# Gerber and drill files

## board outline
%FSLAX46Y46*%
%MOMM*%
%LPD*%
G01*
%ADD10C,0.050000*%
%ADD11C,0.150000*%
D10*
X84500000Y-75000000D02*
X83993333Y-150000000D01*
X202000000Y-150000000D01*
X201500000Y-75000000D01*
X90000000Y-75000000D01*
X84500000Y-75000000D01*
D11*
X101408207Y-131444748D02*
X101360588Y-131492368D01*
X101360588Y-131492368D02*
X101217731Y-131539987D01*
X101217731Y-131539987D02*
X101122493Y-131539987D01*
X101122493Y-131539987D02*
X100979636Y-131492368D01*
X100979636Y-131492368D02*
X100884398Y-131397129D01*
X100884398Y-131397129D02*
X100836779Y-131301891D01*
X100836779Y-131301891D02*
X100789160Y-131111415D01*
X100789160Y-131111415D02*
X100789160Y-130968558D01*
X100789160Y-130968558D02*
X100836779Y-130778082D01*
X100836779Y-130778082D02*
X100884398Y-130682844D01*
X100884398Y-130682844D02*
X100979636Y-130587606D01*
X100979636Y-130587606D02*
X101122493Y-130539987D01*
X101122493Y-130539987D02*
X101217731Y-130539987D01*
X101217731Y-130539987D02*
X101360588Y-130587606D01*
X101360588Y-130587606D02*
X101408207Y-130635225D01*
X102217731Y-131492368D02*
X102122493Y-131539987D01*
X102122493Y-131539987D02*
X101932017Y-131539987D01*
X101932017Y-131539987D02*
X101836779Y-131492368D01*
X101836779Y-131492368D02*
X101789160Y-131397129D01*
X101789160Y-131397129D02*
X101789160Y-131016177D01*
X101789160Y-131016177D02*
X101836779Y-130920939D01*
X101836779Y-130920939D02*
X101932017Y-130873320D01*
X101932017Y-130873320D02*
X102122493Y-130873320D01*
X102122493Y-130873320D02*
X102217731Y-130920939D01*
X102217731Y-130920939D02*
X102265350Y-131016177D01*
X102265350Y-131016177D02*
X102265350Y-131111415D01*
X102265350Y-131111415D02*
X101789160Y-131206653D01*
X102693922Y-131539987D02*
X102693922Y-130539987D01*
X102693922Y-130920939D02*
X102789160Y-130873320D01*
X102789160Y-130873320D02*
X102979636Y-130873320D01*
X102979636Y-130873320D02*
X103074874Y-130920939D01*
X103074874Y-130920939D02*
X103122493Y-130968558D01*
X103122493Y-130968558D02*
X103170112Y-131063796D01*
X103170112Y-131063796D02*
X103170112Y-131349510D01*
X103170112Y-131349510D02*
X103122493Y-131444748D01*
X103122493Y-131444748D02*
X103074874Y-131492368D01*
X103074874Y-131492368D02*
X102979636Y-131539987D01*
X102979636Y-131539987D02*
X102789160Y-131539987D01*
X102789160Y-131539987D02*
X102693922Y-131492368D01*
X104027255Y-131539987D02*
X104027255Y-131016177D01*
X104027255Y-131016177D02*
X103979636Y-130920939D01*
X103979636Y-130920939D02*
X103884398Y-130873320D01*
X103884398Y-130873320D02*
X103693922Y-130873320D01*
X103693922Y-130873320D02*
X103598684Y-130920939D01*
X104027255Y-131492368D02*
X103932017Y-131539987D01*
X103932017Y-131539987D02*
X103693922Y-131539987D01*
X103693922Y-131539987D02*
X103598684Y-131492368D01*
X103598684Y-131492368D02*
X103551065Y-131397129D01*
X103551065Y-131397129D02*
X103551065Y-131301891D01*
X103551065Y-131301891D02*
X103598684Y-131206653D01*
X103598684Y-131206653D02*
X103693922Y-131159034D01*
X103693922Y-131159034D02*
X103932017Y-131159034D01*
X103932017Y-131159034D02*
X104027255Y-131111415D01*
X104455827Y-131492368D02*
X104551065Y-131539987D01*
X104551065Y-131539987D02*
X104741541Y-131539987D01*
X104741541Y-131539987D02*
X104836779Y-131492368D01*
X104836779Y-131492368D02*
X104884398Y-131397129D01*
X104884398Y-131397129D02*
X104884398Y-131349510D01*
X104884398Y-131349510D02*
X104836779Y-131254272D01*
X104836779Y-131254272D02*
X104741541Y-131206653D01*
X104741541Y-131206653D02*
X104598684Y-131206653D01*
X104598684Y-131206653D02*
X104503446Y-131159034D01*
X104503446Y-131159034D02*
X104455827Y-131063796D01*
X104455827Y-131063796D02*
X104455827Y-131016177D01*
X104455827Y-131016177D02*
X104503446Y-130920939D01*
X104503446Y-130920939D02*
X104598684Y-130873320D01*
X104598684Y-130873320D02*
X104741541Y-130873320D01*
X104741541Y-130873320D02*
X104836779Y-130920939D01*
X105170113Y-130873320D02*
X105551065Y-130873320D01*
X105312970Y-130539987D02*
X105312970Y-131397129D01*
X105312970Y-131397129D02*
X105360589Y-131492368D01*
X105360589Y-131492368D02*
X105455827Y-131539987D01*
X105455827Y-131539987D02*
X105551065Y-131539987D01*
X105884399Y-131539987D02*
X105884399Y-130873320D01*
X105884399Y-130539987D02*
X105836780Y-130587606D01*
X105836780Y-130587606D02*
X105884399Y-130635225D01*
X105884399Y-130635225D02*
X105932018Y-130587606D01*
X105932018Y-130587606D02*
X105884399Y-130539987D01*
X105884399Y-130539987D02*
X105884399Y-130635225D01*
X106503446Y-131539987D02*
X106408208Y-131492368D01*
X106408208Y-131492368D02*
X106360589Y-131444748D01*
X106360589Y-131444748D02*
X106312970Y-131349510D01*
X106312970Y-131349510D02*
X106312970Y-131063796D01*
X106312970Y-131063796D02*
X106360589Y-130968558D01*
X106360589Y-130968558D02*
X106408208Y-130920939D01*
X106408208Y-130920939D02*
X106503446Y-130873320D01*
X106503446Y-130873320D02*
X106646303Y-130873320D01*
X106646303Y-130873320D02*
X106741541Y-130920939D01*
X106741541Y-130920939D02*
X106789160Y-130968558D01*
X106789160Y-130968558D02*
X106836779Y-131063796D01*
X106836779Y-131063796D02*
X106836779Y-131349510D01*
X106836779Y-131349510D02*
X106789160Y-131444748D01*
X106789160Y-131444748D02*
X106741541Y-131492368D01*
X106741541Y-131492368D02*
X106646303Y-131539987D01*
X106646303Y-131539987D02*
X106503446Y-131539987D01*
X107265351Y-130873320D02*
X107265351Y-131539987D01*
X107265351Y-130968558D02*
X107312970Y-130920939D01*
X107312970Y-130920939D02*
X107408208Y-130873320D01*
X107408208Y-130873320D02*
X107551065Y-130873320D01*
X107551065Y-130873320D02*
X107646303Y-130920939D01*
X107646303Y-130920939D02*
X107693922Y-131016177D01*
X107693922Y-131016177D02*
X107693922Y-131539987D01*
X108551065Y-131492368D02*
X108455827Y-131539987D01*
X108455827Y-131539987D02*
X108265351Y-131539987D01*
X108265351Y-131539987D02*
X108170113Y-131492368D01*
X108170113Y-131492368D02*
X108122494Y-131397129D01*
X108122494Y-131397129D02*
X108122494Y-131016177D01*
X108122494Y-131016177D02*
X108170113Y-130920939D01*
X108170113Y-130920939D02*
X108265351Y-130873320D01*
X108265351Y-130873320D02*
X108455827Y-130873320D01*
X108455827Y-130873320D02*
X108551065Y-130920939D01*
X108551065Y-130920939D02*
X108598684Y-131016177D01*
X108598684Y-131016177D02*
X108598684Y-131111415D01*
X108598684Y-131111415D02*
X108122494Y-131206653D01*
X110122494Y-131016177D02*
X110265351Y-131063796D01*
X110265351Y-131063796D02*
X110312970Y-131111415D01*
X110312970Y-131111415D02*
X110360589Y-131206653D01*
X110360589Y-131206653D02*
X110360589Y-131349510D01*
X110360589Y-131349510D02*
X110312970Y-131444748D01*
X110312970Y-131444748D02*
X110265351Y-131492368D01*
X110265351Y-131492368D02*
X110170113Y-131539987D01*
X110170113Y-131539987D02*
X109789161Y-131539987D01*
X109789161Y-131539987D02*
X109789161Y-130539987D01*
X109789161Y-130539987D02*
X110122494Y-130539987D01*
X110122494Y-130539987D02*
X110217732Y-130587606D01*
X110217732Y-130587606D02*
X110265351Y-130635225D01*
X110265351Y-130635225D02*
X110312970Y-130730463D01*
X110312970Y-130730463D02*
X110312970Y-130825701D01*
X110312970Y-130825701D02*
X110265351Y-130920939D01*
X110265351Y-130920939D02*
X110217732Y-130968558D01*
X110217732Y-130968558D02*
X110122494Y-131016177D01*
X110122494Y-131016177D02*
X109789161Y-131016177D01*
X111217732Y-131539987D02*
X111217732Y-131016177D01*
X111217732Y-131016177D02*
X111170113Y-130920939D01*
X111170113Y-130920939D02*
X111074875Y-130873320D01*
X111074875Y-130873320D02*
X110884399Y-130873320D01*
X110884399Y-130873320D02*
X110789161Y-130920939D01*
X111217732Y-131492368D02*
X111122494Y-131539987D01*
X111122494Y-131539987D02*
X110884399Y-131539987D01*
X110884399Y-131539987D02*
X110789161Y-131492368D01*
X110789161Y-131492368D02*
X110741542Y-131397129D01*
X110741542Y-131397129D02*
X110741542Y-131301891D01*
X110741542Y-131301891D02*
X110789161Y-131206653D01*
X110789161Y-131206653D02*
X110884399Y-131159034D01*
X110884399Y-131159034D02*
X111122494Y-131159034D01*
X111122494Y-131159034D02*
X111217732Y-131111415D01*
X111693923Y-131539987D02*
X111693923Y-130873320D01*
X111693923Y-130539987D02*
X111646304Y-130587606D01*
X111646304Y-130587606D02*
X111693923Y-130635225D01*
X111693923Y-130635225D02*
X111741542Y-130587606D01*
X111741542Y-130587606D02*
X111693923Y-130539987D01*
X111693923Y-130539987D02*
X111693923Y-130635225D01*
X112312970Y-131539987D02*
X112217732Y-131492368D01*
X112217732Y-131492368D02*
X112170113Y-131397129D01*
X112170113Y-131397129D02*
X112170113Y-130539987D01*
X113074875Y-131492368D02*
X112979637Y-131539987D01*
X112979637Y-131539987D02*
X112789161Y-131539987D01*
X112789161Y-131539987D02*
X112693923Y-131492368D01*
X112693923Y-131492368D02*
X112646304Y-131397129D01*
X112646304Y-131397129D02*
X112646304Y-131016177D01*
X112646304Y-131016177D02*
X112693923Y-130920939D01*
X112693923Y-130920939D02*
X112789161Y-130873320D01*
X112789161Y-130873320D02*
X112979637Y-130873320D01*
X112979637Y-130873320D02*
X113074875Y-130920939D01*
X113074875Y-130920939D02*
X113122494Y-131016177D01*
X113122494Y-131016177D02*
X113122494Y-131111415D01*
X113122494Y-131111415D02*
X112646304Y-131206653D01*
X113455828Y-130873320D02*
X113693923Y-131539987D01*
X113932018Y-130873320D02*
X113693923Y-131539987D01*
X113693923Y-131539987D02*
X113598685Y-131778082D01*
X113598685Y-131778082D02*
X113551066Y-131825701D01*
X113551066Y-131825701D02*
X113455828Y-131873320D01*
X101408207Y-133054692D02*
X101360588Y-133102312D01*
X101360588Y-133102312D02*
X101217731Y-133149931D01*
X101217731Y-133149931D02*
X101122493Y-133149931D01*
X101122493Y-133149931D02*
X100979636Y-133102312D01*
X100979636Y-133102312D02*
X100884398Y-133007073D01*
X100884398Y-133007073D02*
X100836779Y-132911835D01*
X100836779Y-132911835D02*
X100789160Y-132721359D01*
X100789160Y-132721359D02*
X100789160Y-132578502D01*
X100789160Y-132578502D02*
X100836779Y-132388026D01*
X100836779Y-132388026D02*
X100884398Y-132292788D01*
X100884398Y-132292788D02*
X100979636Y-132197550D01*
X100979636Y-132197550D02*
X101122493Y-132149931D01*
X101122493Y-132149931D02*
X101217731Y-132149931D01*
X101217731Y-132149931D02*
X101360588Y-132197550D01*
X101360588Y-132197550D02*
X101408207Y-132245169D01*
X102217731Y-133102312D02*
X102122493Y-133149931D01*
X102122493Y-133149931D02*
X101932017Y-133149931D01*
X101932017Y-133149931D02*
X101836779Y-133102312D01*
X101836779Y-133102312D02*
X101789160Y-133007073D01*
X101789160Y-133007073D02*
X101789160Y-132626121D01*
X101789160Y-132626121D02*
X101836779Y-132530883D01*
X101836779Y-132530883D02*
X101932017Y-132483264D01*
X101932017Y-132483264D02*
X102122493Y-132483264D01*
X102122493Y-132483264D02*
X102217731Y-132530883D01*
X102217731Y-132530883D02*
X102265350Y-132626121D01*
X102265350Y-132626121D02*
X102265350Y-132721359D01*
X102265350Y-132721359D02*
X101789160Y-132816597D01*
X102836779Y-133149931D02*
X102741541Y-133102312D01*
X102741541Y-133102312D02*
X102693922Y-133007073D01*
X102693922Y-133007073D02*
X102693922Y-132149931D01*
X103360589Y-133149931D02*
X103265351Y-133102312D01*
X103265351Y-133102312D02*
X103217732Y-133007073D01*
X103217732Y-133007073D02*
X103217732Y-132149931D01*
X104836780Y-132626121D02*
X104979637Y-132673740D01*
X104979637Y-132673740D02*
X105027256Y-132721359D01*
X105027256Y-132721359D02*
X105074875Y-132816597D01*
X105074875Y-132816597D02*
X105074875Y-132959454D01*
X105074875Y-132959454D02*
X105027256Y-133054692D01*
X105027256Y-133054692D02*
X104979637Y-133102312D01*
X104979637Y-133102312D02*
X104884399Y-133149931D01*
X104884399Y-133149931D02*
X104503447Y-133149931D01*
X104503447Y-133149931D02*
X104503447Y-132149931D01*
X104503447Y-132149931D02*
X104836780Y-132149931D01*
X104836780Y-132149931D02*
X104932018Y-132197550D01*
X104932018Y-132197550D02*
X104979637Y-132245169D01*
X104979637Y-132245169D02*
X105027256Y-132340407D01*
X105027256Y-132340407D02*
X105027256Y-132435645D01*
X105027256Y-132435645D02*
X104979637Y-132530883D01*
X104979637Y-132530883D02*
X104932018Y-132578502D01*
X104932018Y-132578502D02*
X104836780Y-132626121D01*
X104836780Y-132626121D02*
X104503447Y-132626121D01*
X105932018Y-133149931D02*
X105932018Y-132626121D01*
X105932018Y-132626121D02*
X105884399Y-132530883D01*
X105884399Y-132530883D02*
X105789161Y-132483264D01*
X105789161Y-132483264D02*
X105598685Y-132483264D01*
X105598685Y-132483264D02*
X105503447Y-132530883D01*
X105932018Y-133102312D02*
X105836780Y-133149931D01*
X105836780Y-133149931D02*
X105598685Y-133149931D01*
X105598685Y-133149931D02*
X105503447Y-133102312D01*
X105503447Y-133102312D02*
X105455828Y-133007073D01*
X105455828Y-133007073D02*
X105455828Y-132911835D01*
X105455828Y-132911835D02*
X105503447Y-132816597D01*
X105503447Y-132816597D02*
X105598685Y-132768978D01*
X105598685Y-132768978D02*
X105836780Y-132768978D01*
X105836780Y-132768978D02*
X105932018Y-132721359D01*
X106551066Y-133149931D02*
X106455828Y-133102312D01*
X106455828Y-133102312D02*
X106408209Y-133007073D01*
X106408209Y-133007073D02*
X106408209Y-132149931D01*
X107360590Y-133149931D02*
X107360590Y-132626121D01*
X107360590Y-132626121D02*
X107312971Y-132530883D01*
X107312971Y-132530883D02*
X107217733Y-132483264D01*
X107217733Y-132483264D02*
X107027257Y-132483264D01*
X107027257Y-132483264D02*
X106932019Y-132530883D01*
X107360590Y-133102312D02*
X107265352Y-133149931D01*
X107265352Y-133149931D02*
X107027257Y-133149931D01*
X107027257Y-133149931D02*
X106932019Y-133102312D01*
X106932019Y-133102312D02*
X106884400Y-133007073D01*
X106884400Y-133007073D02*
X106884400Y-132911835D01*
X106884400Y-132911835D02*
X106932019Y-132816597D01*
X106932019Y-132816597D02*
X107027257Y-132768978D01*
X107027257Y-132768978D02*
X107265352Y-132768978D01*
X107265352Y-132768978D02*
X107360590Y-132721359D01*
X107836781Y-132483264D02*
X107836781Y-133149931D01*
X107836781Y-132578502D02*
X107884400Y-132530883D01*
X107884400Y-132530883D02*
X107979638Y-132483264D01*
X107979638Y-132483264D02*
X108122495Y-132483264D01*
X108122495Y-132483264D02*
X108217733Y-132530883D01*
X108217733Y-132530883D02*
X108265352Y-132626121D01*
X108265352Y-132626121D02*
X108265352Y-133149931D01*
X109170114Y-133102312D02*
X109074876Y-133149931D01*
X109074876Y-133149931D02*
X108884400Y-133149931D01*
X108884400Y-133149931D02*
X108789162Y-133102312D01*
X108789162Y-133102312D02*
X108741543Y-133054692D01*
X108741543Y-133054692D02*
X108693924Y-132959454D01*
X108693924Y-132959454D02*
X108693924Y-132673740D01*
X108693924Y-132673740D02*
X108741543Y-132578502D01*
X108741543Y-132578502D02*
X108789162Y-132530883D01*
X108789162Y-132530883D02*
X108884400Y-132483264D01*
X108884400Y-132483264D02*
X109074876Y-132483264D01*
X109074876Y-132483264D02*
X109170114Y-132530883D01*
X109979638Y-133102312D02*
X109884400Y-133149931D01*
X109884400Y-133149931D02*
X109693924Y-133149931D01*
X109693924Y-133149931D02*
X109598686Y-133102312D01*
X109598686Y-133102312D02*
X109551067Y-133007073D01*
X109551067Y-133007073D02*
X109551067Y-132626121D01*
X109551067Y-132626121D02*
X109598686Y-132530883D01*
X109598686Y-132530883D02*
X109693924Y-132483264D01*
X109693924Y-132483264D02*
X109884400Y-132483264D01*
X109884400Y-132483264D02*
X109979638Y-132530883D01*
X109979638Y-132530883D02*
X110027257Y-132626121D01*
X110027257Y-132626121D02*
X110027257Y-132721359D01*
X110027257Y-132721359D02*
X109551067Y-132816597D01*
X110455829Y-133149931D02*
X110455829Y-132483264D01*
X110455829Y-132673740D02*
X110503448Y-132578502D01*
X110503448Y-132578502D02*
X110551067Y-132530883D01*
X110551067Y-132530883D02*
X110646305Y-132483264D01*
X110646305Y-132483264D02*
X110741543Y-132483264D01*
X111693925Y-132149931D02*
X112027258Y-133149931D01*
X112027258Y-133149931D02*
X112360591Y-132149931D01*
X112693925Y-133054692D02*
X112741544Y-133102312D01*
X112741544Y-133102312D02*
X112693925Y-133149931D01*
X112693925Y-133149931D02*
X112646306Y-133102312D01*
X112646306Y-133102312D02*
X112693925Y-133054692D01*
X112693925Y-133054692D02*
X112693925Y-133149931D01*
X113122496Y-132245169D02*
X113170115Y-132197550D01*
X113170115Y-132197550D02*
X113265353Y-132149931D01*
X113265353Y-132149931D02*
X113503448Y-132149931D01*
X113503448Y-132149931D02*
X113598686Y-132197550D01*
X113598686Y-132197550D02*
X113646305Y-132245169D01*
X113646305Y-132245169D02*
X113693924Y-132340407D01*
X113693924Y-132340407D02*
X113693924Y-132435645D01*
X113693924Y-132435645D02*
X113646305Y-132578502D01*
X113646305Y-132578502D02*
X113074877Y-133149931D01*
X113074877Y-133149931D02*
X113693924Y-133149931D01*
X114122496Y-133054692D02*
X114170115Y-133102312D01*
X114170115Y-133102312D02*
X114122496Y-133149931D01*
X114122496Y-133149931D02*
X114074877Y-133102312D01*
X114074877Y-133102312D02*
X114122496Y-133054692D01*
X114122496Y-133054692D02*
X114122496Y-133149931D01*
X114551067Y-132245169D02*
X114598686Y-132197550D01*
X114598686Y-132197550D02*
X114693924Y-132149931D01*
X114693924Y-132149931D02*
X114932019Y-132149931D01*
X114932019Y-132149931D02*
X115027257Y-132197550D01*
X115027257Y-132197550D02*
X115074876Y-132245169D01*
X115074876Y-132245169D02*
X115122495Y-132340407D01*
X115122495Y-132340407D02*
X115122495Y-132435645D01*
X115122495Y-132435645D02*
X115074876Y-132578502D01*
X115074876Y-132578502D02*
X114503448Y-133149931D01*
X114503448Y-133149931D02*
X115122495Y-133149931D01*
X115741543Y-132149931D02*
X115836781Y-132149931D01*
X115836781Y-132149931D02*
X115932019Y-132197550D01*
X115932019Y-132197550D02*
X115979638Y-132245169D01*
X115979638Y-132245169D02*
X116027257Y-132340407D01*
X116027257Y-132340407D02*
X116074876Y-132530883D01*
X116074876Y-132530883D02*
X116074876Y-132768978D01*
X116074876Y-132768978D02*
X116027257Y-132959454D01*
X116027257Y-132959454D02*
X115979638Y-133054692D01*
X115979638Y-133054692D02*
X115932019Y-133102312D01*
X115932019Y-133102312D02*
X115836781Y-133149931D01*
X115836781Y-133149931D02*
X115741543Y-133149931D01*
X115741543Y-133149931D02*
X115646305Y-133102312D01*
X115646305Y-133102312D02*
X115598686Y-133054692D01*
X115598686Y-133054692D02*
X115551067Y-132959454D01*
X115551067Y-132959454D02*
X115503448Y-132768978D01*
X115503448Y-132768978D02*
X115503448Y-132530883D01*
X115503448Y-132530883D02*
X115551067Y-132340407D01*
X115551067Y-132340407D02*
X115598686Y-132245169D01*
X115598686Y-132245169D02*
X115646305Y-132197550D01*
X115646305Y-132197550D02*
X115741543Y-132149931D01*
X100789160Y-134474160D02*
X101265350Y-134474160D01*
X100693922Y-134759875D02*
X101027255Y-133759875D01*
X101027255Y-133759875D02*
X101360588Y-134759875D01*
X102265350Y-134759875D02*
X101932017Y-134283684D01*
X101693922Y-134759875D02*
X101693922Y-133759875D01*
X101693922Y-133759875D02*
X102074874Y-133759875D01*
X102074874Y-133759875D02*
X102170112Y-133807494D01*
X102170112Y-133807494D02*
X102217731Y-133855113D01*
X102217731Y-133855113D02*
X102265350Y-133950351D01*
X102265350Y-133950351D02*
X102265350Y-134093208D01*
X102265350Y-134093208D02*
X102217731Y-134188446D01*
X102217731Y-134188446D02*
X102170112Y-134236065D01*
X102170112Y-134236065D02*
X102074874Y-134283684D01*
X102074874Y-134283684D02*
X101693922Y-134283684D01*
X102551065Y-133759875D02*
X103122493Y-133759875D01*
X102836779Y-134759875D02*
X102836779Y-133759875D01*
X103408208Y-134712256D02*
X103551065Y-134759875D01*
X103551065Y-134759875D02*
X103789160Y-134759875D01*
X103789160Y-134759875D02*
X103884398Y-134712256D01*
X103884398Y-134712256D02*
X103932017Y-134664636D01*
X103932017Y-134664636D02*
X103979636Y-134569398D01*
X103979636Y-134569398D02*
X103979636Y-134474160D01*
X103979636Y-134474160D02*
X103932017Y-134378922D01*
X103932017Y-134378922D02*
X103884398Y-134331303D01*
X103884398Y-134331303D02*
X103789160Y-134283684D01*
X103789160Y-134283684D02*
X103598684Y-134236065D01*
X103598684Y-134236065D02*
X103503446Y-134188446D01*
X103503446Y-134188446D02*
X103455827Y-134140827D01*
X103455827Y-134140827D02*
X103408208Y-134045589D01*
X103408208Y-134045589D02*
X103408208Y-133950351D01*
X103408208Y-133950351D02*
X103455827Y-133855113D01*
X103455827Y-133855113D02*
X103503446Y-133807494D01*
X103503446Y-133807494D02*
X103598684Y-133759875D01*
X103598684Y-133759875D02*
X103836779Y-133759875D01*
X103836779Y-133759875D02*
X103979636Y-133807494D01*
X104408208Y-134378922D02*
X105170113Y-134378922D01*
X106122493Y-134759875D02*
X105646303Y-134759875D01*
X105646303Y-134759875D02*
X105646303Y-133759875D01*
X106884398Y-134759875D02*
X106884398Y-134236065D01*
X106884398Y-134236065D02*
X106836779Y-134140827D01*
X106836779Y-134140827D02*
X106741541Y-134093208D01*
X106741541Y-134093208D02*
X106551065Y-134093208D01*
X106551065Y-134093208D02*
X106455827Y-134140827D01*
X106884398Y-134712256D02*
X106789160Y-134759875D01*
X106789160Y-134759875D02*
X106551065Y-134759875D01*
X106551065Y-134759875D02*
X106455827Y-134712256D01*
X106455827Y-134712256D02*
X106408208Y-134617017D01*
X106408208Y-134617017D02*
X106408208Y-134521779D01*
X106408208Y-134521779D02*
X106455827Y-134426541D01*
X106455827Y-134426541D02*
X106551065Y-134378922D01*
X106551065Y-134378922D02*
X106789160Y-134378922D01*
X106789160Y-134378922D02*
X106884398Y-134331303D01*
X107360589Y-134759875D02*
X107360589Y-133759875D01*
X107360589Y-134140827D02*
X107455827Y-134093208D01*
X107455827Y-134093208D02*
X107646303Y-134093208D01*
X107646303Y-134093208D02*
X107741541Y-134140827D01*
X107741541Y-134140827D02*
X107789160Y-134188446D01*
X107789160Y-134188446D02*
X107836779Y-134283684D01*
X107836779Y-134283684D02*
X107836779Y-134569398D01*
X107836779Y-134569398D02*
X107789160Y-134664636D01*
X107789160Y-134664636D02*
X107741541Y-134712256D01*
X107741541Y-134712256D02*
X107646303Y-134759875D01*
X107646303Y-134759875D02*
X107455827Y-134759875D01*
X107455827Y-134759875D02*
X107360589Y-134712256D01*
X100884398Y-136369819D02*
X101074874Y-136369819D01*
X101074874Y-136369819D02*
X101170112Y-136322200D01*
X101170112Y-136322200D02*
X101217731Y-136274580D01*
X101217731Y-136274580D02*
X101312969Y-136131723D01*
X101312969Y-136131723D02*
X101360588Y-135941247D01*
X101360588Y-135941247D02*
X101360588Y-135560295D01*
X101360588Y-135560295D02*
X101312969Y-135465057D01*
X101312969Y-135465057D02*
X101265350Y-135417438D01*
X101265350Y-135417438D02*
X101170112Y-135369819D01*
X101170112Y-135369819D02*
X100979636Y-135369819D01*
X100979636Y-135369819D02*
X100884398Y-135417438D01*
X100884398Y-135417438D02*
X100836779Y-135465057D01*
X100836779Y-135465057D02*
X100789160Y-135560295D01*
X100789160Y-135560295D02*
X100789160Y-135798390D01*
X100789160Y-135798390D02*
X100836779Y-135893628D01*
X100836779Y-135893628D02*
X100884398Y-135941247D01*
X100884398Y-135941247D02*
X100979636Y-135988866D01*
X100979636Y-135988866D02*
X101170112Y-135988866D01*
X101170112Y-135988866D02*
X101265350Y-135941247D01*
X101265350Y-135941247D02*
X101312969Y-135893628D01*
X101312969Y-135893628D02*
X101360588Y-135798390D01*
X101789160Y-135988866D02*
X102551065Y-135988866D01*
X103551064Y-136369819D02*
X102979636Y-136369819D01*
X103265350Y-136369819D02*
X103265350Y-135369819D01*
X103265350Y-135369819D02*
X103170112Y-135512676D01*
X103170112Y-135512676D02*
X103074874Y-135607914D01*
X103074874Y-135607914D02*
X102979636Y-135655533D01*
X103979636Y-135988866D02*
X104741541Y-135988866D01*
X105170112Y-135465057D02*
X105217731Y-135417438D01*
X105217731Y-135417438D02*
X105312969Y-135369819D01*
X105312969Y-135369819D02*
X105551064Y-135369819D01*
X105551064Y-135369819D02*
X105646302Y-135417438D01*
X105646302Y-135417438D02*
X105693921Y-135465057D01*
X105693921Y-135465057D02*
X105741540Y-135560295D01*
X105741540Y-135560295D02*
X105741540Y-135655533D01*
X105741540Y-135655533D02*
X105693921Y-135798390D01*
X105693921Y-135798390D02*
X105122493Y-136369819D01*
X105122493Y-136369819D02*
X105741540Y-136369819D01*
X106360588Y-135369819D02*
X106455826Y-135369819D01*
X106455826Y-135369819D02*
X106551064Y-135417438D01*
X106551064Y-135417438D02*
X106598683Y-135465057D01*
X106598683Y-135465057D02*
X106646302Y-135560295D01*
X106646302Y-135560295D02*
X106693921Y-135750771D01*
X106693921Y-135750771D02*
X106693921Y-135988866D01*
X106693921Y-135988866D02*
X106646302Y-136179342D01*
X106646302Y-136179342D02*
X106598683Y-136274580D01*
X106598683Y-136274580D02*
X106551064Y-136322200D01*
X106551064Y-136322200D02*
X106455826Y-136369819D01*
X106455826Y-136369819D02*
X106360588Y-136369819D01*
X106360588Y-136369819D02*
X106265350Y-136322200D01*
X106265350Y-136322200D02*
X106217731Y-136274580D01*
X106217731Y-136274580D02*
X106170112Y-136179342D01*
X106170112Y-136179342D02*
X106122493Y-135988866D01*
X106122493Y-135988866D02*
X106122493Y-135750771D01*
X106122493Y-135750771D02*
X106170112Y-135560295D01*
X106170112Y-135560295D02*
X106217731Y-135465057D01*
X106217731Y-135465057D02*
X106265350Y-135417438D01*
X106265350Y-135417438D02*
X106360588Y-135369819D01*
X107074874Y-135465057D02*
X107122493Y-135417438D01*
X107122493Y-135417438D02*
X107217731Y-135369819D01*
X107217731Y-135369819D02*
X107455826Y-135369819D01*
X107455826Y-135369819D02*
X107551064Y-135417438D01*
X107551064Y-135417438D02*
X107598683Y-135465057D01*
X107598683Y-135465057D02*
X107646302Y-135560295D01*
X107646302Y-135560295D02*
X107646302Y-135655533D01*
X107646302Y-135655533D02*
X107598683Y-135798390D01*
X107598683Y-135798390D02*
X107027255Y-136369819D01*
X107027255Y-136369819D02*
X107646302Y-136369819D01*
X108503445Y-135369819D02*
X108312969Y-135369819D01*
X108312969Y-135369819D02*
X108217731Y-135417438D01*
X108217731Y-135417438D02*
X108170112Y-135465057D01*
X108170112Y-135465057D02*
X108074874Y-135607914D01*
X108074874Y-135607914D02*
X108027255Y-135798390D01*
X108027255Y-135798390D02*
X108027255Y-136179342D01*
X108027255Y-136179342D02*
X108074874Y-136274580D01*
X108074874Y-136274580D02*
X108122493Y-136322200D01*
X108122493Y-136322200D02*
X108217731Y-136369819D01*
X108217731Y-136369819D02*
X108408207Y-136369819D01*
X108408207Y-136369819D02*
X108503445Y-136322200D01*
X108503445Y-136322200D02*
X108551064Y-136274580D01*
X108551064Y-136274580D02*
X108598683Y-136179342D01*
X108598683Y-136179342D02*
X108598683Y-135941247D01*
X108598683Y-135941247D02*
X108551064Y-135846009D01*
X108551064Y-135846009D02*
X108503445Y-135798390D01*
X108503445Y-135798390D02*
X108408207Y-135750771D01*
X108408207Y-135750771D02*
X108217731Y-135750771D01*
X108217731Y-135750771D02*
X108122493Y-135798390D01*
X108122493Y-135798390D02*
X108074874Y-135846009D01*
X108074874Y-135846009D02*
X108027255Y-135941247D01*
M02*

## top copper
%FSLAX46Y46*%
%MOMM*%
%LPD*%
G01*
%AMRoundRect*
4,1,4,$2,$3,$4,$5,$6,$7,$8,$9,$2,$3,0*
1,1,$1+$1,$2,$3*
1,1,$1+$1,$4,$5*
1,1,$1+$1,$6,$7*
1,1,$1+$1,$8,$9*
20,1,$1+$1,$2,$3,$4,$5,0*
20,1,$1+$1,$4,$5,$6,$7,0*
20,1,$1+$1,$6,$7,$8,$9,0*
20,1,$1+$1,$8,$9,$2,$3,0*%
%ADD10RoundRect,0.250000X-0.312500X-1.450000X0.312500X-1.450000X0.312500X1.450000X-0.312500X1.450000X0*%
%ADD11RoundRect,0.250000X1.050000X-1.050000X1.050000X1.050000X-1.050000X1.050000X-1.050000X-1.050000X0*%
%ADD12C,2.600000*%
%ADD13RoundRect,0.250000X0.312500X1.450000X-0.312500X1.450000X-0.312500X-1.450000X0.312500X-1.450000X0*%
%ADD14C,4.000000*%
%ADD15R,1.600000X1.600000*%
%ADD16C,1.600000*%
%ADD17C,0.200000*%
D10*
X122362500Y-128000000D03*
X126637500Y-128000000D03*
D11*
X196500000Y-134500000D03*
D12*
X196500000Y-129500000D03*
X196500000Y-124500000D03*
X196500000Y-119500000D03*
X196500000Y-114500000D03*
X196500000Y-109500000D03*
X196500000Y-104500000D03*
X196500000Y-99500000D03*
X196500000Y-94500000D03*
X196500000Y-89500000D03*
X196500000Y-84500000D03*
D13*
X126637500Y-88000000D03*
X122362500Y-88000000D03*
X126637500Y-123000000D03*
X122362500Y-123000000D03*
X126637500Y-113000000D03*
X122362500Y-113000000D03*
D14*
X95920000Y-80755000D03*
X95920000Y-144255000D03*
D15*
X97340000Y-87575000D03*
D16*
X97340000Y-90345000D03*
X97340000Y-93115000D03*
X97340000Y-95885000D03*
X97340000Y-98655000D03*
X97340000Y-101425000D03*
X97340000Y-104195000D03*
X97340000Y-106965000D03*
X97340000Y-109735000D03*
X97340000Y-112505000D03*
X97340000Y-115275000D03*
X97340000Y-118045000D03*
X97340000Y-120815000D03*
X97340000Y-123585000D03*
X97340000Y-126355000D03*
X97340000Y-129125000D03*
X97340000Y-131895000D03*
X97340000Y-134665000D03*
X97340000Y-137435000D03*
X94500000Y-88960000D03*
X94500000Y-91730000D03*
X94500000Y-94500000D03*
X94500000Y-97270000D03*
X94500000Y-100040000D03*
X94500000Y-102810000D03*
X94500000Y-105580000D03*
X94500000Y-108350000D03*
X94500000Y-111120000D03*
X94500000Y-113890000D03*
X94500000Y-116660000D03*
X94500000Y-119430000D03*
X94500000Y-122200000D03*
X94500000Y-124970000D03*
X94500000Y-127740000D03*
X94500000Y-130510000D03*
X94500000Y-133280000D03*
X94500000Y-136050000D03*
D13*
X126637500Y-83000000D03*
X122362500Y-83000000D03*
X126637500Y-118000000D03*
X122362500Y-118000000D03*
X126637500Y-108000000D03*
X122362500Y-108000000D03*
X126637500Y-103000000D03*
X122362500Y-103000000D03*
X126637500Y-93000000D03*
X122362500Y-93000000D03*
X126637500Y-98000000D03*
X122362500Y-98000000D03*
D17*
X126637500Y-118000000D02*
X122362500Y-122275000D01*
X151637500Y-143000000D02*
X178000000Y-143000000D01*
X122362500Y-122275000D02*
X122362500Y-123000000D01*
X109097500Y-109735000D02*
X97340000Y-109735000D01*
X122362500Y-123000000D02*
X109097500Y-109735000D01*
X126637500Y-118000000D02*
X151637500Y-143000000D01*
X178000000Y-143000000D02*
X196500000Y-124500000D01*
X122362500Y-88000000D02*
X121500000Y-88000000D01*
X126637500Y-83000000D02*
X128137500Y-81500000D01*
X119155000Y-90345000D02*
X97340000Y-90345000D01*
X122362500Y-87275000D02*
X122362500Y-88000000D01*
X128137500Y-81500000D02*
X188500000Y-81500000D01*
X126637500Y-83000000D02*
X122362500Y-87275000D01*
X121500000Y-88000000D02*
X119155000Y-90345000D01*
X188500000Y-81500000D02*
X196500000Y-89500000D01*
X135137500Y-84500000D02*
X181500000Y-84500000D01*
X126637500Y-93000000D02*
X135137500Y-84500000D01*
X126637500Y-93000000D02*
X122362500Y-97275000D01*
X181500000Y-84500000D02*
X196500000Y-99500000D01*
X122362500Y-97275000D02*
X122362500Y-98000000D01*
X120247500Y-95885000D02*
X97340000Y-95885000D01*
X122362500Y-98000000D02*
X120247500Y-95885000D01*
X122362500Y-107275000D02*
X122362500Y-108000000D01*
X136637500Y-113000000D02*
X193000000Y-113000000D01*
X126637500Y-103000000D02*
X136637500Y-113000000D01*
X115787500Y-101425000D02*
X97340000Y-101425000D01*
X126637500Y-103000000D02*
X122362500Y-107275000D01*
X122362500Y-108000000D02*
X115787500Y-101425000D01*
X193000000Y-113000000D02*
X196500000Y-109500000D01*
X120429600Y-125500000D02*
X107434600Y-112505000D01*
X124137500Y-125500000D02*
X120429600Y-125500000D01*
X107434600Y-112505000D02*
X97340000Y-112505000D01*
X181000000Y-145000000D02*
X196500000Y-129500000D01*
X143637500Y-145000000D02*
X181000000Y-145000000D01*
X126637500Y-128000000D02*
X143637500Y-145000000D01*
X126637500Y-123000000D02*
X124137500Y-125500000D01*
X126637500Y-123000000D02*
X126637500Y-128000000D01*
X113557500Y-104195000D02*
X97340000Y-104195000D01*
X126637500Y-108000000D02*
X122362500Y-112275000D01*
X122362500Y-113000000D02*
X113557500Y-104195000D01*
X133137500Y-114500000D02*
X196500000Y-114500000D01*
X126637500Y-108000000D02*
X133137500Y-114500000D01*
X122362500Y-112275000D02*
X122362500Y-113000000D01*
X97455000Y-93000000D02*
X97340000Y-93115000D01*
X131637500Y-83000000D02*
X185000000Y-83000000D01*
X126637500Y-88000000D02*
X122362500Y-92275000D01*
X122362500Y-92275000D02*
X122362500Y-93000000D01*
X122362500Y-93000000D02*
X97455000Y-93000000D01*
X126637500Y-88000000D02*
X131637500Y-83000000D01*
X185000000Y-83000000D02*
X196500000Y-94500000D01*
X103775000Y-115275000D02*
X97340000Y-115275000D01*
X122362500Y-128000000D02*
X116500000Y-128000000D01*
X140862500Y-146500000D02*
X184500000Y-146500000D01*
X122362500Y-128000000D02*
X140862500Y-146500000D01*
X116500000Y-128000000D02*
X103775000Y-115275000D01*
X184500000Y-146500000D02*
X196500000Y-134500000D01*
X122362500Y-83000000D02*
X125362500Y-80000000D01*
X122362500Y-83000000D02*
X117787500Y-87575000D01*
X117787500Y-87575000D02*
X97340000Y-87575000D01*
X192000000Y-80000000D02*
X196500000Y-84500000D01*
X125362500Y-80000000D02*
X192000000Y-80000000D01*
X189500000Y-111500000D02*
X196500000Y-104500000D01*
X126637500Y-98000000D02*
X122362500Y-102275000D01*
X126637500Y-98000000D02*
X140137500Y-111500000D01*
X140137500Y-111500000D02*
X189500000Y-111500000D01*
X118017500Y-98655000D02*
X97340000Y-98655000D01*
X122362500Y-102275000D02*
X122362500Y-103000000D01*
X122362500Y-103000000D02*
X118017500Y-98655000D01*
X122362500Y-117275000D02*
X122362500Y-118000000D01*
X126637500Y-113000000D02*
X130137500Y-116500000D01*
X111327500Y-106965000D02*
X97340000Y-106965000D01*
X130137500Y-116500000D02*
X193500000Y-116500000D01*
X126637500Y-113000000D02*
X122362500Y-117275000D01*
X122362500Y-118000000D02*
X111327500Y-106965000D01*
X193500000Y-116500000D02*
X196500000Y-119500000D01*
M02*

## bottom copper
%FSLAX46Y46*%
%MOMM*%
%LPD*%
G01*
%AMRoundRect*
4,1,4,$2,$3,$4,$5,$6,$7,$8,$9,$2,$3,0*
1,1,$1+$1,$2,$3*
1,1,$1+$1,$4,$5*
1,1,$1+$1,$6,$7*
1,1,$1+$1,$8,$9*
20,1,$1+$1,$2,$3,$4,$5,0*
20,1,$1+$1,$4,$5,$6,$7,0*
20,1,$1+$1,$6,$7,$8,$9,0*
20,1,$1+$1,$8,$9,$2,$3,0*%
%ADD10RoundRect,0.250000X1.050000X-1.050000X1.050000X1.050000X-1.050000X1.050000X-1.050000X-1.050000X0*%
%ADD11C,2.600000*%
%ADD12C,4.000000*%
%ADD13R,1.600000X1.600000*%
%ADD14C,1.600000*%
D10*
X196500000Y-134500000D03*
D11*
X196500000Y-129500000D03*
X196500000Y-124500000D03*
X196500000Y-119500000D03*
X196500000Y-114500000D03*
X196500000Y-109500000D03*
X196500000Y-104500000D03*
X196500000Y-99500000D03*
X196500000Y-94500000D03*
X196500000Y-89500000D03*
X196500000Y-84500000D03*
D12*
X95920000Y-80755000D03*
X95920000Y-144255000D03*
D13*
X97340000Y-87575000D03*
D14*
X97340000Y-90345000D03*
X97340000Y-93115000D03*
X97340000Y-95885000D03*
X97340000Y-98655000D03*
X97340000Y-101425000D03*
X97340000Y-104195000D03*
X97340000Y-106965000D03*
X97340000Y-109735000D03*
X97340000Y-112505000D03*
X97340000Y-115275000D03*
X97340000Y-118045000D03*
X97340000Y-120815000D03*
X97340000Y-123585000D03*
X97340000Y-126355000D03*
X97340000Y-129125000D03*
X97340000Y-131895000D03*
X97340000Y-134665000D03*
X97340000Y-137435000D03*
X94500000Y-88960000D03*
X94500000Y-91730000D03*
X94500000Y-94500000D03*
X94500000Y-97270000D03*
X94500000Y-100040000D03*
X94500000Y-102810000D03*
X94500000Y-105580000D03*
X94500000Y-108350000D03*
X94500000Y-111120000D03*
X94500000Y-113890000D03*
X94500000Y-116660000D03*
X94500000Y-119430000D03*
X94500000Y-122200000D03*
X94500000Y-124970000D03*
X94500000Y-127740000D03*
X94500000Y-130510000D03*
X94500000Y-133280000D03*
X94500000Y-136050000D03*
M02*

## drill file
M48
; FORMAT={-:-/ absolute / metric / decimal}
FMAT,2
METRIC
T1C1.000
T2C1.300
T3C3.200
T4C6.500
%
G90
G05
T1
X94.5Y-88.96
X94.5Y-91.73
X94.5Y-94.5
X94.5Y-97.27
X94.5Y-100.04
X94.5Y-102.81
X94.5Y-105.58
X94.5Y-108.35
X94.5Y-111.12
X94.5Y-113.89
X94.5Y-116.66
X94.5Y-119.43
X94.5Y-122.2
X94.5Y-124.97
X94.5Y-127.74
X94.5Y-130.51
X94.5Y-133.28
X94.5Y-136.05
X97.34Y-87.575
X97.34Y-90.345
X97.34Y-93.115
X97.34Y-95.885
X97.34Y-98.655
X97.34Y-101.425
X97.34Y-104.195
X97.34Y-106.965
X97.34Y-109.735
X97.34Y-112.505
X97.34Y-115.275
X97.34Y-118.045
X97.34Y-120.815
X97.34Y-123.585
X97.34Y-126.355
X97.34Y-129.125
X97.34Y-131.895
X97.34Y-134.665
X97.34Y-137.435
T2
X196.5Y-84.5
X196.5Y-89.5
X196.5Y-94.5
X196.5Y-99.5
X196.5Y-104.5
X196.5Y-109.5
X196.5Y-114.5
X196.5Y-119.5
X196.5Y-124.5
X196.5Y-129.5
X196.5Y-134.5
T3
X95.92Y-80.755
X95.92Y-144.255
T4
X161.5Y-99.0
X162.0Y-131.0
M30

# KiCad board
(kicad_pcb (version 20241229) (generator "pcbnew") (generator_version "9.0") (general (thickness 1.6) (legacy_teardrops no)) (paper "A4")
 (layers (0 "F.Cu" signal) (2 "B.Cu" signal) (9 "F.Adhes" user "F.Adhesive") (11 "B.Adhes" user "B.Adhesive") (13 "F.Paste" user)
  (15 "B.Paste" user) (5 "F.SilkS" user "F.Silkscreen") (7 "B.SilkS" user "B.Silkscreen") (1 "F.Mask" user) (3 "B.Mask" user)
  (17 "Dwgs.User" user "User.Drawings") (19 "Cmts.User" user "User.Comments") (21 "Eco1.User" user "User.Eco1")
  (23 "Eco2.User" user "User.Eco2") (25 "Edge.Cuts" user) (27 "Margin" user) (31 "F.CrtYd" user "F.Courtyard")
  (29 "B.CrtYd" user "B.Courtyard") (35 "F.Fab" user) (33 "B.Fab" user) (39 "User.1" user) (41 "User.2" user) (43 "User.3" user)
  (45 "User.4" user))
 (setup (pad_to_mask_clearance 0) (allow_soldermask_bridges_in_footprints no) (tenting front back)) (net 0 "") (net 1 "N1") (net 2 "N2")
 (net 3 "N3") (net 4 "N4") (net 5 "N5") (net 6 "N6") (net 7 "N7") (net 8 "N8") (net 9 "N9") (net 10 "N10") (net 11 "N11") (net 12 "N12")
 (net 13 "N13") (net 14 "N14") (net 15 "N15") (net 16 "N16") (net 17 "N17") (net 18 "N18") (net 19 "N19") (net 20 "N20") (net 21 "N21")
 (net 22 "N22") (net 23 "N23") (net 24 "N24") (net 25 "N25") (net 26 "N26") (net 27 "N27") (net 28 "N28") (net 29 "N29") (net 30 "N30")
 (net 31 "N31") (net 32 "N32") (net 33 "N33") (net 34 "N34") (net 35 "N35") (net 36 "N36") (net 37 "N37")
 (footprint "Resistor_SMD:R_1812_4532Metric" (layer "F.Cu") (at 124.5 128)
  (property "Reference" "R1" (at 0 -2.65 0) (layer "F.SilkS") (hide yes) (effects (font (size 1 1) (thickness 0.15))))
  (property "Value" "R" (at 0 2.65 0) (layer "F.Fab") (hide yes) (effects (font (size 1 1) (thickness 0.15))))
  (pad "1" smd roundrect (at -2.1375 0) (size 1.125 3.4) (layers "F.Cu" "F.Mask" "F.Paste") (roundrect_rratio 0.222222) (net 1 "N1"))
  (pad "2" smd roundrect (at 2.1375 0) (size 1.125 3.4) (layers "F.Cu" "F.Mask" "F.Paste") (roundrect_rratio 0.222222) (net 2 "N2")))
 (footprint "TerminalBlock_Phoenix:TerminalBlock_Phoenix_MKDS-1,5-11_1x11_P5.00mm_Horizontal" (layer "F.Cu") (at 196.5 134.5 90)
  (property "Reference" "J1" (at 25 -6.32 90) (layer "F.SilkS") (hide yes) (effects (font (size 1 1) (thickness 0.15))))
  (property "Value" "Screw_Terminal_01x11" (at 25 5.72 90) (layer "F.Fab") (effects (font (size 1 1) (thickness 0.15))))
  (pad "1" thru_hole roundrect (at 0 0 90) (size 2.6 2.6) (drill 1.3) (layers "*.Cu" "*.Mask") (remove_unused_layers no)
   (roundrect_rratio 0.096154) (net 1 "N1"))
  (pad "2" thru_hole circle (at 5 0 90) (size 2.6 2.6) (drill 1.3) (layers "*.Cu" "*.Mask") (remove_unused_layers no) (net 2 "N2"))
  (pad "3" thru_hole circle (at 10 0 90) (size 2.6 2.6) (drill 1.3) (layers "*.Cu" "*.Mask") (remove_unused_layers no) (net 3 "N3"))
  (pad "4" thru_hole circle (at 15 0 90) (size 2.6 2.6) (drill 1.3) (layers "*.Cu" "*.Mask") (remove_unused_layers no) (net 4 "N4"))
  (pad "5" thru_hole circle (at 20 0 90) (size 2.6 2.6) (drill 1.3) (layers "*.Cu" "*.Mask") (remove_unused_layers no) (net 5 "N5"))
  (pad "6" thru_hole circle (at 25 0 90) (size 2.6 2.6) (drill 1.3) (layers "*.Cu" "*.Mask") (remove_unused_layers no) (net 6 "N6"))
  (pad "7" thru_hole circle (at 30 0 90) (size 2.6 2.6) (drill 1.3) (layers "*.Cu" "*.Mask") (remove_unused_layers no) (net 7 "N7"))
  (pad "8" thru_hole circle (at 35 0 90) (size 2.6 2.6) (drill 1.3) (layers "*.Cu" "*.Mask") (remove_unused_layers no) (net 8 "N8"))
  (pad "9" thru_hole circle (at 40 0 90) (size 2.6 2.6) (drill 1.3) (layers "*.Cu" "*.Mask") (remove_unused_layers no) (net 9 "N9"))
  (pad "10" thru_hole circle (at 45 0 90) (size 2.6 2.6) (drill 1.3) (layers "*.Cu" "*.Mask") (remove_unused_layers no) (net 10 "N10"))
  (pad "11" thru_hole circle (at 50 0 90) (size 2.6 2.6) (drill 1.3) (layers "*.Cu" "*.Mask") (remove_unused_layers no) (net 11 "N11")))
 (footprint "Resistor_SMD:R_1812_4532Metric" (layer "F.Cu") (at 124.5 88 180)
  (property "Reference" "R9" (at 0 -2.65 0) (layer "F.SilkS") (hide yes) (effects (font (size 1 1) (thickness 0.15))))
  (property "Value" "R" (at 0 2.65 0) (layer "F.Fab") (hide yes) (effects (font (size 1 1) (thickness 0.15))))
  (pad "1" smd roundrect (at -2.1375 0 180) (size 1.125 3.4) (layers "F.Cu" "F.Mask" "F.Paste") (roundrect_rratio 0.222222) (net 9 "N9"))
  (pad "2" smd roundrect (at 2.1375 0 180) (size 1.125 3.4) (layers "F.Cu" "F.Mask" "F.Paste") (roundrect_rratio 0.222222) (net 10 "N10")))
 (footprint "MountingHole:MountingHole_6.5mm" (layer "F.Cu") (at 161.5 99)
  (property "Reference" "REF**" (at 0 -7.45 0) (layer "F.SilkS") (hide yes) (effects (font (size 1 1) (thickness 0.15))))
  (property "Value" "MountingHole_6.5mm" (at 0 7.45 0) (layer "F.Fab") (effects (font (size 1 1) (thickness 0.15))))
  (pad "" np_thru_hole circle (at 0 0) (size 6.5 6.5) (drill 6.5) (layers "*.Cu" "*.Mask")))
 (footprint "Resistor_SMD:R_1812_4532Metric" (layer "F.Cu") (at 124.5 123 180)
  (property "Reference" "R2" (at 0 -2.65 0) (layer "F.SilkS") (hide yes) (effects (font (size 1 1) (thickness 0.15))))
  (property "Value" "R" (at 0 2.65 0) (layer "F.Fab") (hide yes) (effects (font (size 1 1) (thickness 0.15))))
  (pad "1" smd roundrect (at -2.1375 0 180) (size 1.125 3.4) (layers "F.Cu" "F.Mask" "F.Paste") (roundrect_rratio 0.222222) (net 2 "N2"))
  (pad "2" smd roundrect (at 2.1375 0 180) (size 1.125 3.4) (layers "F.Cu" "F.Mask" "F.Paste") (roundrect_rratio 0.222222) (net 3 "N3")))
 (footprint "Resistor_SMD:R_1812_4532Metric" (layer "F.Cu") (at 124.5 113 180)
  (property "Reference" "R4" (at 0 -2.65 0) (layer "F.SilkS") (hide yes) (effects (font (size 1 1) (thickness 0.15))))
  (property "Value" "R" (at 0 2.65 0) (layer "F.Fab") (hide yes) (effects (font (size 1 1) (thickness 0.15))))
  (pad "1" smd roundrect (at -2.1375 0 180) (size 1.125 3.4) (layers "F.Cu" "F.Mask" "F.Paste") (roundrect_rratio 0.222222) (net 4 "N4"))
  (pad "2" smd roundrect (at 2.1375 0 180) (size 1.125 3.4) (layers "F.Cu" "F.Mask" "F.Paste") (roundrect_rratio 0.222222) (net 5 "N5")))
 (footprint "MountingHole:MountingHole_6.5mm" (layer "F.Cu") (at 162 131)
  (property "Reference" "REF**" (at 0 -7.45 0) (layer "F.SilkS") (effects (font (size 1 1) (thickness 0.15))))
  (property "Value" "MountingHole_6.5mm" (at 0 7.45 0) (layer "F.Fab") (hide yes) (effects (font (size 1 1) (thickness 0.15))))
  (pad "" np_thru_hole circle (at 0 0) (size 6.5 6.5) (drill 6.5) (layers "*.Cu" "*.Mask")))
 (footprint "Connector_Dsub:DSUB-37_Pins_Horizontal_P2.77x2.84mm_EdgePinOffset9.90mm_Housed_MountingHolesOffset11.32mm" (layer "F.Cu")
  (at 97.34 87.575 -90)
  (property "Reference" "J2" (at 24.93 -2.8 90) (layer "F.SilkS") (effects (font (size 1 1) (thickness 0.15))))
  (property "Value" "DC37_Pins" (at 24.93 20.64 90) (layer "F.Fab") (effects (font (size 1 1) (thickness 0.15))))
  (pad "0" thru_hole circle (at -6.82 1.42 270) (size 4 4) (drill 3.2) (layers "*.Cu" "*.Mask") (remove_unused_layers no))
  (pad "0" thru_hole circle (at 56.68 1.42 270) (size 4 4) (drill 3.2) (layers "*.Cu" "*.Mask") (remove_unused_layers no))
  (pad "1" thru_hole rect (at 0 0 270) (size 1.6 1.6) (drill 1) (layers "*.Cu" "*.Mask") (remove_unused_layers no) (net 11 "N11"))
  (pad "2" thru_hole circle (at 2.77 0 270) (size 1.6 1.6) (drill 1) (layers "*.Cu" "*.Mask") (remove_unused_layers no) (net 10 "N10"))
  (pad "3" thru_hole circle (at 5.54 0 270) (size 1.6 1.6) (drill 1) (layers "*.Cu" "*.Mask") (remove_unused_layers no) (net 9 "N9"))
  (pad "4" thru_hole circle (at 8.31 0 270) (size 1.6 1.6) (drill 1) (layers "*.Cu" "*.Mask") (remove_unused_layers no) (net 8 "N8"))
  (pad "5" thru_hole circle (at 11.08 0 270) (size 1.6 1.6) (drill 1) (layers "*.Cu" "*.Mask") (remove_unused_layers no) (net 7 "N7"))
  (pad "6" thru_hole circle (at 13.85 0 270) (size 1.6 1.6) (drill 1) (layers "*.Cu" "*.Mask") (remove_unused_layers no) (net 6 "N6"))
  (pad "7" thru_hole circle (at 16.62 0 270) (size 1.6 1.6) (drill 1) (layers "*.Cu" "*.Mask") (remove_unused_layers no) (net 5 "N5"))
  (pad "8" thru_hole circle (at 19.39 0 270) (size 1.6 1.6) (drill 1) (layers "*.Cu" "*.Mask") (remove_unused_layers no) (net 4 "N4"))
  (pad "9" thru_hole circle (at 22.16 0 270) (size 1.6 1.6) (drill 1) (layers "*.Cu" "*.Mask") (remove_unused_layers no) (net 3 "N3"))
  (pad "10" thru_hole circle (at 24.93 0 270) (size 1.6 1.6) (drill 1) (layers "*.Cu" "*.Mask") (remove_unused_layers no) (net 2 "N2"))
  (pad "11" thru_hole circle (at 27.7 0 270) (size 1.6 1.6) (drill 1) (layers "*.Cu" "*.Mask") (remove_unused_layers no) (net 1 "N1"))
  (pad "12" thru_hole circle (at 30.47 0 270) (size 1.6 1.6) (drill 1) (layers "*.Cu" "*.Mask") (remove_unused_layers no) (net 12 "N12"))
  (pad "13" thru_hole circle (at 33.24 0 270) (size 1.6 1.6) (drill 1) (layers "*.Cu" "*.Mask") (remove_unused_layers no) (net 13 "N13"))
  (pad "14" thru_hole circle (at 36.01 0 270) (size 1.6 1.6) (drill 1) (layers "*.Cu" "*.Mask") (remove_unused_layers no) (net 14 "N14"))
  (pad "15" thru_hole circle (at 38.78 0 270) (size 1.6 1.6) (drill 1) (layers "*.Cu" "*.Mask") (remove_unused_layers no) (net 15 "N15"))
  (pad "16" thru_hole circle (at 41.55 0 270) (size 1.6 1.6) (drill 1) (layers "*.Cu" "*.Mask") (remove_unused_layers no) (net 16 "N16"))
  (pad "17" thru_hole circle (at 44.32 0 270) (size 1.6 1.6) (drill 1) (layers "*.Cu" "*.Mask") (remove_unused_layers no) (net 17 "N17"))
  (pad "18" thru_hole circle (at 47.09 0 270) (size 1.6 1.6) (drill 1) (layers "*.Cu" "*.Mask") (remove_unused_layers no) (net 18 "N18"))
  (pad "19" thru_hole circle (at 49.86 0 270) (size 1.6 1.6) (drill 1) (layers "*.Cu" "*.Mask") (remove_unused_layers no) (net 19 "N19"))
  (pad "20" thru_hole circle (at 1.385 2.84 270) (size 1.6 1.6) (drill 1) (layers "*.Cu" "*.Mask") (remove_unused_layers no) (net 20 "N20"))
  (pad "21" thru_hole circle (at 4.155 2.84 270) (size 1.6 1.6) (drill 1) (layers "*.Cu" "*.Mask") (remove_unused_layers no) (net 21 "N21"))
  (pad "22" thru_hole circle (at 6.925 2.84 270) (size 1.6 1.6) (drill 1) (layers "*.Cu" "*.Mask") (remove_unused_layers no) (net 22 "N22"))
  (pad "23" thru_hole circle (at 9.695 2.84 270) (size 1.6 1.6) (drill 1) (layers "*.Cu" "*.Mask") (remove_unused_layers no) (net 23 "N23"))
  (pad "24" thru_hole circle (at 12.465 2.84 270) (size 1.6 1.6) (drill 1) (layers "*.Cu" "*.Mask") (remove_unused_layers no) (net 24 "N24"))
  (pad "25" thru_hole circle (at 15.235 2.84 270) (size 1.6 1.6) (drill 1) (layers "*.Cu" "*.Mask") (remove_unused_layers no) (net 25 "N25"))
  (pad "26" thru_hole circle (at 18.005 2.84 270) (size 1.6 1.6) (drill 1) (layers "*.Cu" "*.Mask") (remove_unused_layers no) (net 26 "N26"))
  (pad "27" thru_hole circle (at 20.775 2.84 270) (size 1.6 1.6) (drill 1) (layers "*.Cu" "*.Mask") (remove_unused_layers no) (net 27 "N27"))
  (pad "28" thru_hole circle (at 23.545 2.84 270) (size 1.6 1.6) (drill 1) (layers "*.Cu" "*.Mask") (remove_unused_layers no) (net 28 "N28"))
  (pad "29" thru_hole circle (at 26.315 2.84 270) (size 1.6 1.6) (drill 1) (layers "*.Cu" "*.Mask") (remove_unused_layers no) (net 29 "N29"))
  (pad "30" thru_hole circle (at 29.085 2.84 270) (size 1.6 1.6) (drill 1) (layers "*.Cu" "*.Mask") (remove_unused_layers no) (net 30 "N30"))
  (pad "31" thru_hole circle (at 31.855 2.84 270) (size 1.6 1.6) (drill 1) (layers "*.Cu" "*.Mask") (remove_unused_layers no) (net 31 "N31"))
  (pad "32" thru_hole circle (at 34.625 2.84 270) (size 1.6 1.6) (drill 1) (layers "*.Cu" "*.Mask") (remove_unused_layers no) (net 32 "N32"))
  (pad "33" thru_hole circle (at 37.395 2.84 270) (size 1.6 1.6) (drill 1) (layers "*.Cu" "*.Mask") (remove_unused_layers no) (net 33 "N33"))
  (pad "34" thru_hole circle (at 40.165 2.84 270) (size 1.6 1.6) (drill 1) (layers "*.Cu" "*.Mask") (remove_unused_layers no) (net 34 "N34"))
  (pad "35" thru_hole circle (at 42.935 2.84 270) (size 1.6 1.6) (drill 1) (layers "*.Cu" "*.Mask") (remove_unused_layers no) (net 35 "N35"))
  (pad "36" thru_hole circle (at 45.705 2.84 270) (size 1.6 1.6) (drill 1) (layers "*.Cu" "*.Mask") (remove_unused_layers no) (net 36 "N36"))
  (pad "37" thru_hole circle (at 48.475 2.84 270) (size 1.6 1.6) (drill 1) (layers "*.Cu" "*.Mask") (remove_unused_layers no) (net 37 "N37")))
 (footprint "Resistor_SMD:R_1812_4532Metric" (layer "F.Cu") (at 124.5 83 180)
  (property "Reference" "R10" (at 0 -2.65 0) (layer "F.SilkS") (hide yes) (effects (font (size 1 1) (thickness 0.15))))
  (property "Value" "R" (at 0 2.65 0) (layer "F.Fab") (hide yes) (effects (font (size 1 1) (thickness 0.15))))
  (pad "1" smd roundrect (at -2.1375 0 180) (size 1.125 3.4) (layers "F.Cu" "F.Mask" "F.Paste") (roundrect_rratio 0.222222) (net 10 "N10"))
  (pad "2" smd roundrect (at 2.1375 0 180) (size 1.125 3.4) (layers "F.Cu" "F.Mask" "F.Paste") (roundrect_rratio 0.222222) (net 11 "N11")))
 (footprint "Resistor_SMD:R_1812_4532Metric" (layer "F.Cu") (at 124.5 118 180)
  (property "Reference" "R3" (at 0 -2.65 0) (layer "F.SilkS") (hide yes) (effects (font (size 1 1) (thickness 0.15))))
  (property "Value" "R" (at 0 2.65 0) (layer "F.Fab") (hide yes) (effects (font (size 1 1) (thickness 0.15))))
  (pad "1" smd roundrect (at -2.1375 0 180) (size 1.125 3.4) (layers "F.Cu" "F.Mask" "F.Paste") (roundrect_rratio 0.222222) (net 3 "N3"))
  (pad "2" smd roundrect (at 2.1375 0 180) (size 1.125 3.4) (layers "F.Cu" "F.Mask" "F.Paste") (roundrect_rratio 0.222222) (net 4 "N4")))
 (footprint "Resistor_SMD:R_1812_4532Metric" (layer "F.Cu") (at 124.5 108 180)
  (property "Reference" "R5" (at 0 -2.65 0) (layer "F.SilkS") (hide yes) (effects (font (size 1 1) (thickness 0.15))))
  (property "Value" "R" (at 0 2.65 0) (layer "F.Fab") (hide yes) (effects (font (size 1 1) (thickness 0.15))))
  (pad "1" smd roundrect (at -2.1375 0 180) (size 1.125 3.4) (layers "F.Cu" "F.Mask" "F.Paste") (roundrect_rratio 0.222222) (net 5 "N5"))
  (pad "2" smd roundrect (at 2.1375 0 180) (size 1.125 3.4) (layers "F.Cu" "F.Mask" "F.Paste") (roundrect_rratio 0.222222) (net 6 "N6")))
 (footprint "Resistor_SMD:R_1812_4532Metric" (layer "F.Cu") (at 124.5 103 180)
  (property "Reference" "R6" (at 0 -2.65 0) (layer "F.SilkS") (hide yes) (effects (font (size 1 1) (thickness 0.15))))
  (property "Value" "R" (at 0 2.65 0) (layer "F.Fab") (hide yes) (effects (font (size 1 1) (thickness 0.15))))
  (pad "1" smd roundrect (at -2.1375 0 180) (size 1.125 3.4) (layers "F.Cu" "F.Mask" "F.Paste") (roundrect_rratio 0.222222) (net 6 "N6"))
  (pad "2" smd roundrect (at 2.1375 0 180) (size 1.125 3.4) (layers "F.Cu" "F.Mask" "F.Paste") (roundrect_rratio 0.222222) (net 7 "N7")))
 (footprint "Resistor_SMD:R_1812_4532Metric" (layer "F.Cu") (at 124.5 93 180)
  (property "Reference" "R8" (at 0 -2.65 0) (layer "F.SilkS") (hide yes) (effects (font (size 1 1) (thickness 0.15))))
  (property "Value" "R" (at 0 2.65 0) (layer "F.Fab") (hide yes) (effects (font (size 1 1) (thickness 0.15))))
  (pad "1" smd roundrect (at -2.1375 0 180) (size 1.125 3.4) (layers "F.Cu" "F.Mask" "F.Paste") (roundrect_rratio 0.222222) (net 8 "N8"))
  (pad "2" smd roundrect (at 2.1375 0 180) (size 1.125 3.4) (layers "F.Cu" "F.Mask" "F.Paste") (roundrect_rratio 0.222222) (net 9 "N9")))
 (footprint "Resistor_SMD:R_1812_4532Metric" (layer "F.Cu") (at 124.5 98 180)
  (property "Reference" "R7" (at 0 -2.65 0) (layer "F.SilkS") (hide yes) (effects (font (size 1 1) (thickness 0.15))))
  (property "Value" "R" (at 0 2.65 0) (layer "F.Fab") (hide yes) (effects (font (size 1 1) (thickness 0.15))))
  (pad "1" smd roundrect (at -2.1375 0 180) (size 1.125 3.4) (layers "F.Cu" "F.Mask" "F.Paste") (roundrect_rratio 0.222222) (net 7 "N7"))
  (pad "2" smd roundrect (at 2.1375 0 180) (size 1.125 3.4) (layers "F.Cu" "F.Mask" "F.Paste") (roundrect_rratio 0.222222) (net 8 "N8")))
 (gr_poly
  (pts (xy 84.5 75) (xy 83.993333 150) (xy 202 150) (xy 201.5 75) (xy 90 75)) (stroke (width 0.05) (type solid)) (fill no)
  (layer "Edge.Cuts"))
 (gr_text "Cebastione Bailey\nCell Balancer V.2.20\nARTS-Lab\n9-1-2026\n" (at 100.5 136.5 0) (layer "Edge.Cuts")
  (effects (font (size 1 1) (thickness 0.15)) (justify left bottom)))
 (segment (start 126.6375 118) (end 122.3625 122.275) (width 0.2) (layer "F.Cu") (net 3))
 (segment (start 151.6375 143) (end 178 143) (width 0.2) (layer "F.Cu") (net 3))
 (segment (start 122.3625 122.275) (end 122.3625 123) (width 0.2) (layer "F.Cu") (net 3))
 (segment (start 109.0975 109.735) (end 97.34 109.735) (width 0.2) (layer "F.Cu") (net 3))
 (segment (start 122.3625 123) (end 109.0975 109.735) (width 0.2) (layer "F.Cu") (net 3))
 (segment (start 126.6375 118) (end 151.6375 143) (width 0.2) (layer "F.Cu") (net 3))
 (segment (start 178 143) (end 196.5 124.5) (width 0.2) (layer "F.Cu") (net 3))
 (segment (start 122.3625 88) (end 121.5 88) (width 0.2) (layer "F.Cu") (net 10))
 (segment (start 126.6375 83) (end 128.1375 81.5) (width 0.2) (layer "F.Cu") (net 10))
 (segment (start 119.155 90.345) (end 97.34 90.345) (width 0.2) (layer "F.Cu") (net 10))
 (segment (start 122.3625 87.275) (end 122.3625 88) (width 0.2) (layer "F.Cu") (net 10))
 (segment (start 128.1375 81.5) (end 188.5 81.5) (width 0.2) (layer "F.Cu") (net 10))
 (segment (start 126.6375 83) (end 122.3625 87.275) (width 0.2) (layer "F.Cu") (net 10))
 (segment (start 121.5 88) (end 119.155 90.345) (width 0.2) (layer "F.Cu") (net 10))
 (segment (start 188.5 81.5) (end 196.5 89.5) (width 0.2) (layer "F.Cu") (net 10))
 (segment (start 135.1375 84.5) (end 181.5 84.5) (width 0.2) (layer "F.Cu") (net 8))
 (segment (start 126.6375 93) (end 135.1375 84.5) (width 0.2) (layer "F.Cu") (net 8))
 (segment (start 126.6375 93) (end 122.3625 97.275) (width 0.2) (layer "F.Cu") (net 8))
 (segment (start 181.5 84.5) (end 196.5 99.5) (width 0.2) (layer "F.Cu") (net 8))
 (segment (start 122.3625 97.275) (end 122.3625 98) (width 0.2) (layer "F.Cu") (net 8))
 (segment (start 120.2475 95.885) (end 97.34 95.885) (width 0.2) (layer "F.Cu") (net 8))
 (segment (start 122.3625 98) (end 120.2475 95.885) (width 0.2) (layer "F.Cu") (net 8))
 (segment (start 122.3625 107.275) (end 122.3625 108) (width 0.2) (layer "F.Cu") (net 6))
 (segment (start 136.6375 113) (end 193 113) (width 0.2) (layer "F.Cu") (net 6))
 (segment (start 126.6375 103) (end 136.6375 113) (width 0.2) (layer "F.Cu") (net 6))
 (segment (start 115.7875 101.425) (end 97.34 101.425) (width 0.2) (layer "F.Cu") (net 6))
 (segment (start 126.6375 103) (end 122.3625 107.275) (width 0.2) (layer "F.Cu") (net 6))
 (segment (start 122.3625 108) (end 115.7875 101.425) (width 0.2) (layer "F.Cu") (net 6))
 (segment (start 193 113) (end 196.5 109.5) (width 0.2) (layer "F.Cu") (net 6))
 (segment (start 120.4296 125.5) (end 107.4346 112.505) (width 0.2) (layer "F.Cu") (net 2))
 (segment (start 124.1375 125.5) (end 120.4296 125.5) (width 0.2) (layer "F.Cu") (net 2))
 (segment (start 107.4346 112.505) (end 97.34 112.505) (width 0.2) (layer "F.Cu") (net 2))
 (segment (start 181 145) (end 196.5 129.5) (width 0.2) (layer "F.Cu") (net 2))
 (segment (start 143.6375 145) (end 181 145) (width 0.2) (layer "F.Cu") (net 2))
 (segment (start 126.6375 128) (end 143.6375 145) (width 0.2) (layer "F.Cu") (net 2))
 (segment (start 126.6375 123) (end 124.1375 125.5) (width 0.2) (layer "F.Cu") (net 2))
 (segment (start 126.6375 123) (end 126.6375 128) (width 0.2) (layer "F.Cu") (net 2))
 (segment (start 113.5575 104.195) (end 97.34 104.195) (width 0.2) (layer "F.Cu") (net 5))
 (segment (start 126.6375 108) (end 122.3625 112.275) (width 0.2) (layer "F.Cu") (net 5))
 (segment (start 122.3625 113) (end 113.5575 104.195) (width 0.2) (layer "F.Cu") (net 5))
 (segment (start 133.1375 114.5) (end 196.5 114.5) (width 0.2) (layer "F.Cu") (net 5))
 (segment (start 126.6375 108) (end 133.1375 114.5) (width 0.2) (layer "F.Cu") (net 5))
 (segment (start 122.3625 112.275) (end 122.3625 113) (width 0.2) (layer "F.Cu") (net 5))
 (segment (start 97.455 93) (end 97.34 93.115) (width 0.2) (layer "F.Cu") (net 9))
 (segment (start 131.6375 83) (end 185 83) (width 0.2) (layer "F.Cu") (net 9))
 (segment (start 126.6375 88) (end 122.3625 92.275) (width 0.2) (layer "F.Cu") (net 9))
 (segment (start 122.3625 92.275) (end 122.3625 93) (width 0.2) (layer "F.Cu") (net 9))
 (segment (start 122.3625 93) (end 97.455 93) (width 0.2) (layer "F.Cu") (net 9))
 (segment (start 126.6375 88) (end 131.6375 83) (width 0.2) (layer "F.Cu") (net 9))
 (segment (start 185 83) (end 196.5 94.5) (width 0.2) (layer "F.Cu") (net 9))
 (segment (start 103.775 115.275) (end 97.34 115.275) (width 0.2) (layer "F.Cu") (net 1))
 (segment (start 122.3625 128) (end 116.5 128) (width 0.2) (layer "F.Cu") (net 1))
 (segment (start 140.8625 146.5) (end 184.5 146.5) (width 0.2) (layer "F.Cu") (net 1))
 (segment (start 122.3625 128) (end 140.8625 146.5) (width 0.2) (layer "F.Cu") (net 1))
 (segment (start 116.5 128) (end 103.775 115.275) (width 0.2) (layer "F.Cu") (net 1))
 (segment (start 184.5 146.5) (end 196.5 134.5) (width 0.2) (layer "F.Cu") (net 1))
 (segment (start 122.3625 83) (end 125.3625 80) (width 0.2) (layer "F.Cu") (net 11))
 (segment (start 122.3625 83) (end 117.7875 87.575) (width 0.2) (layer "F.Cu") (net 11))
 (segment (start 117.7875 87.575) (end 97.34 87.575) (width 0.2) (layer "F.Cu") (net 11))
 (segment (start 192 80) (end 196.5 84.5) (width 0.2) (layer "F.Cu") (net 11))
 (segment (start 125.3625 80) (end 192 80) (width 0.2) (layer "F.Cu") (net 11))
 (segment (start 189.5 111.5) (end 196.5 104.5) (width 0.2) (layer "F.Cu") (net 7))
 (segment (start 126.6375 98) (end 122.3625 102.275) (width 0.2) (layer "F.Cu") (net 7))
 (segment (start 126.6375 98) (end 140.1375 111.5) (width 0.2) (layer "F.Cu") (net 7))
 (segment (start 140.1375 111.5) (end 189.5 111.5) (width 0.2) (layer "F.Cu") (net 7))
 (segment (start 118.0175 98.655) (end 97.34 98.655) (width 0.2) (layer "F.Cu") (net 7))
 (segment (start 122.3625 102.275) (end 122.3625 103) (width 0.2) (layer "F.Cu") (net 7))
 (segment (start 122.3625 103) (end 118.0175 98.655) (width 0.2) (layer "F.Cu") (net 7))
 (segment (start 122.3625 117.275) (end 122.3625 118) (width 0.2) (layer "F.Cu") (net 4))
 (segment (start 126.6375 113) (end 130.1375 116.5) (width 0.2) (layer "F.Cu") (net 4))
 (segment (start 111.3275 106.965) (end 97.34 106.965) (width 0.2) (layer "F.Cu") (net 4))
 (segment (start 130.1375 116.5) (end 193.5 116.5) (width 0.2) (layer "F.Cu") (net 4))
 (segment (start 126.6375 113) (end 122.3625 117.275) (width 0.2) (layer "F.Cu") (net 4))
 (segment (start 122.3625 118) (end 111.3275 106.965) (width 0.2) (layer "F.Cu") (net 4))
 (segment (start 193.5 116.5) (end 196.5 119.5) (width 0.2) (layer "F.Cu") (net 4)))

